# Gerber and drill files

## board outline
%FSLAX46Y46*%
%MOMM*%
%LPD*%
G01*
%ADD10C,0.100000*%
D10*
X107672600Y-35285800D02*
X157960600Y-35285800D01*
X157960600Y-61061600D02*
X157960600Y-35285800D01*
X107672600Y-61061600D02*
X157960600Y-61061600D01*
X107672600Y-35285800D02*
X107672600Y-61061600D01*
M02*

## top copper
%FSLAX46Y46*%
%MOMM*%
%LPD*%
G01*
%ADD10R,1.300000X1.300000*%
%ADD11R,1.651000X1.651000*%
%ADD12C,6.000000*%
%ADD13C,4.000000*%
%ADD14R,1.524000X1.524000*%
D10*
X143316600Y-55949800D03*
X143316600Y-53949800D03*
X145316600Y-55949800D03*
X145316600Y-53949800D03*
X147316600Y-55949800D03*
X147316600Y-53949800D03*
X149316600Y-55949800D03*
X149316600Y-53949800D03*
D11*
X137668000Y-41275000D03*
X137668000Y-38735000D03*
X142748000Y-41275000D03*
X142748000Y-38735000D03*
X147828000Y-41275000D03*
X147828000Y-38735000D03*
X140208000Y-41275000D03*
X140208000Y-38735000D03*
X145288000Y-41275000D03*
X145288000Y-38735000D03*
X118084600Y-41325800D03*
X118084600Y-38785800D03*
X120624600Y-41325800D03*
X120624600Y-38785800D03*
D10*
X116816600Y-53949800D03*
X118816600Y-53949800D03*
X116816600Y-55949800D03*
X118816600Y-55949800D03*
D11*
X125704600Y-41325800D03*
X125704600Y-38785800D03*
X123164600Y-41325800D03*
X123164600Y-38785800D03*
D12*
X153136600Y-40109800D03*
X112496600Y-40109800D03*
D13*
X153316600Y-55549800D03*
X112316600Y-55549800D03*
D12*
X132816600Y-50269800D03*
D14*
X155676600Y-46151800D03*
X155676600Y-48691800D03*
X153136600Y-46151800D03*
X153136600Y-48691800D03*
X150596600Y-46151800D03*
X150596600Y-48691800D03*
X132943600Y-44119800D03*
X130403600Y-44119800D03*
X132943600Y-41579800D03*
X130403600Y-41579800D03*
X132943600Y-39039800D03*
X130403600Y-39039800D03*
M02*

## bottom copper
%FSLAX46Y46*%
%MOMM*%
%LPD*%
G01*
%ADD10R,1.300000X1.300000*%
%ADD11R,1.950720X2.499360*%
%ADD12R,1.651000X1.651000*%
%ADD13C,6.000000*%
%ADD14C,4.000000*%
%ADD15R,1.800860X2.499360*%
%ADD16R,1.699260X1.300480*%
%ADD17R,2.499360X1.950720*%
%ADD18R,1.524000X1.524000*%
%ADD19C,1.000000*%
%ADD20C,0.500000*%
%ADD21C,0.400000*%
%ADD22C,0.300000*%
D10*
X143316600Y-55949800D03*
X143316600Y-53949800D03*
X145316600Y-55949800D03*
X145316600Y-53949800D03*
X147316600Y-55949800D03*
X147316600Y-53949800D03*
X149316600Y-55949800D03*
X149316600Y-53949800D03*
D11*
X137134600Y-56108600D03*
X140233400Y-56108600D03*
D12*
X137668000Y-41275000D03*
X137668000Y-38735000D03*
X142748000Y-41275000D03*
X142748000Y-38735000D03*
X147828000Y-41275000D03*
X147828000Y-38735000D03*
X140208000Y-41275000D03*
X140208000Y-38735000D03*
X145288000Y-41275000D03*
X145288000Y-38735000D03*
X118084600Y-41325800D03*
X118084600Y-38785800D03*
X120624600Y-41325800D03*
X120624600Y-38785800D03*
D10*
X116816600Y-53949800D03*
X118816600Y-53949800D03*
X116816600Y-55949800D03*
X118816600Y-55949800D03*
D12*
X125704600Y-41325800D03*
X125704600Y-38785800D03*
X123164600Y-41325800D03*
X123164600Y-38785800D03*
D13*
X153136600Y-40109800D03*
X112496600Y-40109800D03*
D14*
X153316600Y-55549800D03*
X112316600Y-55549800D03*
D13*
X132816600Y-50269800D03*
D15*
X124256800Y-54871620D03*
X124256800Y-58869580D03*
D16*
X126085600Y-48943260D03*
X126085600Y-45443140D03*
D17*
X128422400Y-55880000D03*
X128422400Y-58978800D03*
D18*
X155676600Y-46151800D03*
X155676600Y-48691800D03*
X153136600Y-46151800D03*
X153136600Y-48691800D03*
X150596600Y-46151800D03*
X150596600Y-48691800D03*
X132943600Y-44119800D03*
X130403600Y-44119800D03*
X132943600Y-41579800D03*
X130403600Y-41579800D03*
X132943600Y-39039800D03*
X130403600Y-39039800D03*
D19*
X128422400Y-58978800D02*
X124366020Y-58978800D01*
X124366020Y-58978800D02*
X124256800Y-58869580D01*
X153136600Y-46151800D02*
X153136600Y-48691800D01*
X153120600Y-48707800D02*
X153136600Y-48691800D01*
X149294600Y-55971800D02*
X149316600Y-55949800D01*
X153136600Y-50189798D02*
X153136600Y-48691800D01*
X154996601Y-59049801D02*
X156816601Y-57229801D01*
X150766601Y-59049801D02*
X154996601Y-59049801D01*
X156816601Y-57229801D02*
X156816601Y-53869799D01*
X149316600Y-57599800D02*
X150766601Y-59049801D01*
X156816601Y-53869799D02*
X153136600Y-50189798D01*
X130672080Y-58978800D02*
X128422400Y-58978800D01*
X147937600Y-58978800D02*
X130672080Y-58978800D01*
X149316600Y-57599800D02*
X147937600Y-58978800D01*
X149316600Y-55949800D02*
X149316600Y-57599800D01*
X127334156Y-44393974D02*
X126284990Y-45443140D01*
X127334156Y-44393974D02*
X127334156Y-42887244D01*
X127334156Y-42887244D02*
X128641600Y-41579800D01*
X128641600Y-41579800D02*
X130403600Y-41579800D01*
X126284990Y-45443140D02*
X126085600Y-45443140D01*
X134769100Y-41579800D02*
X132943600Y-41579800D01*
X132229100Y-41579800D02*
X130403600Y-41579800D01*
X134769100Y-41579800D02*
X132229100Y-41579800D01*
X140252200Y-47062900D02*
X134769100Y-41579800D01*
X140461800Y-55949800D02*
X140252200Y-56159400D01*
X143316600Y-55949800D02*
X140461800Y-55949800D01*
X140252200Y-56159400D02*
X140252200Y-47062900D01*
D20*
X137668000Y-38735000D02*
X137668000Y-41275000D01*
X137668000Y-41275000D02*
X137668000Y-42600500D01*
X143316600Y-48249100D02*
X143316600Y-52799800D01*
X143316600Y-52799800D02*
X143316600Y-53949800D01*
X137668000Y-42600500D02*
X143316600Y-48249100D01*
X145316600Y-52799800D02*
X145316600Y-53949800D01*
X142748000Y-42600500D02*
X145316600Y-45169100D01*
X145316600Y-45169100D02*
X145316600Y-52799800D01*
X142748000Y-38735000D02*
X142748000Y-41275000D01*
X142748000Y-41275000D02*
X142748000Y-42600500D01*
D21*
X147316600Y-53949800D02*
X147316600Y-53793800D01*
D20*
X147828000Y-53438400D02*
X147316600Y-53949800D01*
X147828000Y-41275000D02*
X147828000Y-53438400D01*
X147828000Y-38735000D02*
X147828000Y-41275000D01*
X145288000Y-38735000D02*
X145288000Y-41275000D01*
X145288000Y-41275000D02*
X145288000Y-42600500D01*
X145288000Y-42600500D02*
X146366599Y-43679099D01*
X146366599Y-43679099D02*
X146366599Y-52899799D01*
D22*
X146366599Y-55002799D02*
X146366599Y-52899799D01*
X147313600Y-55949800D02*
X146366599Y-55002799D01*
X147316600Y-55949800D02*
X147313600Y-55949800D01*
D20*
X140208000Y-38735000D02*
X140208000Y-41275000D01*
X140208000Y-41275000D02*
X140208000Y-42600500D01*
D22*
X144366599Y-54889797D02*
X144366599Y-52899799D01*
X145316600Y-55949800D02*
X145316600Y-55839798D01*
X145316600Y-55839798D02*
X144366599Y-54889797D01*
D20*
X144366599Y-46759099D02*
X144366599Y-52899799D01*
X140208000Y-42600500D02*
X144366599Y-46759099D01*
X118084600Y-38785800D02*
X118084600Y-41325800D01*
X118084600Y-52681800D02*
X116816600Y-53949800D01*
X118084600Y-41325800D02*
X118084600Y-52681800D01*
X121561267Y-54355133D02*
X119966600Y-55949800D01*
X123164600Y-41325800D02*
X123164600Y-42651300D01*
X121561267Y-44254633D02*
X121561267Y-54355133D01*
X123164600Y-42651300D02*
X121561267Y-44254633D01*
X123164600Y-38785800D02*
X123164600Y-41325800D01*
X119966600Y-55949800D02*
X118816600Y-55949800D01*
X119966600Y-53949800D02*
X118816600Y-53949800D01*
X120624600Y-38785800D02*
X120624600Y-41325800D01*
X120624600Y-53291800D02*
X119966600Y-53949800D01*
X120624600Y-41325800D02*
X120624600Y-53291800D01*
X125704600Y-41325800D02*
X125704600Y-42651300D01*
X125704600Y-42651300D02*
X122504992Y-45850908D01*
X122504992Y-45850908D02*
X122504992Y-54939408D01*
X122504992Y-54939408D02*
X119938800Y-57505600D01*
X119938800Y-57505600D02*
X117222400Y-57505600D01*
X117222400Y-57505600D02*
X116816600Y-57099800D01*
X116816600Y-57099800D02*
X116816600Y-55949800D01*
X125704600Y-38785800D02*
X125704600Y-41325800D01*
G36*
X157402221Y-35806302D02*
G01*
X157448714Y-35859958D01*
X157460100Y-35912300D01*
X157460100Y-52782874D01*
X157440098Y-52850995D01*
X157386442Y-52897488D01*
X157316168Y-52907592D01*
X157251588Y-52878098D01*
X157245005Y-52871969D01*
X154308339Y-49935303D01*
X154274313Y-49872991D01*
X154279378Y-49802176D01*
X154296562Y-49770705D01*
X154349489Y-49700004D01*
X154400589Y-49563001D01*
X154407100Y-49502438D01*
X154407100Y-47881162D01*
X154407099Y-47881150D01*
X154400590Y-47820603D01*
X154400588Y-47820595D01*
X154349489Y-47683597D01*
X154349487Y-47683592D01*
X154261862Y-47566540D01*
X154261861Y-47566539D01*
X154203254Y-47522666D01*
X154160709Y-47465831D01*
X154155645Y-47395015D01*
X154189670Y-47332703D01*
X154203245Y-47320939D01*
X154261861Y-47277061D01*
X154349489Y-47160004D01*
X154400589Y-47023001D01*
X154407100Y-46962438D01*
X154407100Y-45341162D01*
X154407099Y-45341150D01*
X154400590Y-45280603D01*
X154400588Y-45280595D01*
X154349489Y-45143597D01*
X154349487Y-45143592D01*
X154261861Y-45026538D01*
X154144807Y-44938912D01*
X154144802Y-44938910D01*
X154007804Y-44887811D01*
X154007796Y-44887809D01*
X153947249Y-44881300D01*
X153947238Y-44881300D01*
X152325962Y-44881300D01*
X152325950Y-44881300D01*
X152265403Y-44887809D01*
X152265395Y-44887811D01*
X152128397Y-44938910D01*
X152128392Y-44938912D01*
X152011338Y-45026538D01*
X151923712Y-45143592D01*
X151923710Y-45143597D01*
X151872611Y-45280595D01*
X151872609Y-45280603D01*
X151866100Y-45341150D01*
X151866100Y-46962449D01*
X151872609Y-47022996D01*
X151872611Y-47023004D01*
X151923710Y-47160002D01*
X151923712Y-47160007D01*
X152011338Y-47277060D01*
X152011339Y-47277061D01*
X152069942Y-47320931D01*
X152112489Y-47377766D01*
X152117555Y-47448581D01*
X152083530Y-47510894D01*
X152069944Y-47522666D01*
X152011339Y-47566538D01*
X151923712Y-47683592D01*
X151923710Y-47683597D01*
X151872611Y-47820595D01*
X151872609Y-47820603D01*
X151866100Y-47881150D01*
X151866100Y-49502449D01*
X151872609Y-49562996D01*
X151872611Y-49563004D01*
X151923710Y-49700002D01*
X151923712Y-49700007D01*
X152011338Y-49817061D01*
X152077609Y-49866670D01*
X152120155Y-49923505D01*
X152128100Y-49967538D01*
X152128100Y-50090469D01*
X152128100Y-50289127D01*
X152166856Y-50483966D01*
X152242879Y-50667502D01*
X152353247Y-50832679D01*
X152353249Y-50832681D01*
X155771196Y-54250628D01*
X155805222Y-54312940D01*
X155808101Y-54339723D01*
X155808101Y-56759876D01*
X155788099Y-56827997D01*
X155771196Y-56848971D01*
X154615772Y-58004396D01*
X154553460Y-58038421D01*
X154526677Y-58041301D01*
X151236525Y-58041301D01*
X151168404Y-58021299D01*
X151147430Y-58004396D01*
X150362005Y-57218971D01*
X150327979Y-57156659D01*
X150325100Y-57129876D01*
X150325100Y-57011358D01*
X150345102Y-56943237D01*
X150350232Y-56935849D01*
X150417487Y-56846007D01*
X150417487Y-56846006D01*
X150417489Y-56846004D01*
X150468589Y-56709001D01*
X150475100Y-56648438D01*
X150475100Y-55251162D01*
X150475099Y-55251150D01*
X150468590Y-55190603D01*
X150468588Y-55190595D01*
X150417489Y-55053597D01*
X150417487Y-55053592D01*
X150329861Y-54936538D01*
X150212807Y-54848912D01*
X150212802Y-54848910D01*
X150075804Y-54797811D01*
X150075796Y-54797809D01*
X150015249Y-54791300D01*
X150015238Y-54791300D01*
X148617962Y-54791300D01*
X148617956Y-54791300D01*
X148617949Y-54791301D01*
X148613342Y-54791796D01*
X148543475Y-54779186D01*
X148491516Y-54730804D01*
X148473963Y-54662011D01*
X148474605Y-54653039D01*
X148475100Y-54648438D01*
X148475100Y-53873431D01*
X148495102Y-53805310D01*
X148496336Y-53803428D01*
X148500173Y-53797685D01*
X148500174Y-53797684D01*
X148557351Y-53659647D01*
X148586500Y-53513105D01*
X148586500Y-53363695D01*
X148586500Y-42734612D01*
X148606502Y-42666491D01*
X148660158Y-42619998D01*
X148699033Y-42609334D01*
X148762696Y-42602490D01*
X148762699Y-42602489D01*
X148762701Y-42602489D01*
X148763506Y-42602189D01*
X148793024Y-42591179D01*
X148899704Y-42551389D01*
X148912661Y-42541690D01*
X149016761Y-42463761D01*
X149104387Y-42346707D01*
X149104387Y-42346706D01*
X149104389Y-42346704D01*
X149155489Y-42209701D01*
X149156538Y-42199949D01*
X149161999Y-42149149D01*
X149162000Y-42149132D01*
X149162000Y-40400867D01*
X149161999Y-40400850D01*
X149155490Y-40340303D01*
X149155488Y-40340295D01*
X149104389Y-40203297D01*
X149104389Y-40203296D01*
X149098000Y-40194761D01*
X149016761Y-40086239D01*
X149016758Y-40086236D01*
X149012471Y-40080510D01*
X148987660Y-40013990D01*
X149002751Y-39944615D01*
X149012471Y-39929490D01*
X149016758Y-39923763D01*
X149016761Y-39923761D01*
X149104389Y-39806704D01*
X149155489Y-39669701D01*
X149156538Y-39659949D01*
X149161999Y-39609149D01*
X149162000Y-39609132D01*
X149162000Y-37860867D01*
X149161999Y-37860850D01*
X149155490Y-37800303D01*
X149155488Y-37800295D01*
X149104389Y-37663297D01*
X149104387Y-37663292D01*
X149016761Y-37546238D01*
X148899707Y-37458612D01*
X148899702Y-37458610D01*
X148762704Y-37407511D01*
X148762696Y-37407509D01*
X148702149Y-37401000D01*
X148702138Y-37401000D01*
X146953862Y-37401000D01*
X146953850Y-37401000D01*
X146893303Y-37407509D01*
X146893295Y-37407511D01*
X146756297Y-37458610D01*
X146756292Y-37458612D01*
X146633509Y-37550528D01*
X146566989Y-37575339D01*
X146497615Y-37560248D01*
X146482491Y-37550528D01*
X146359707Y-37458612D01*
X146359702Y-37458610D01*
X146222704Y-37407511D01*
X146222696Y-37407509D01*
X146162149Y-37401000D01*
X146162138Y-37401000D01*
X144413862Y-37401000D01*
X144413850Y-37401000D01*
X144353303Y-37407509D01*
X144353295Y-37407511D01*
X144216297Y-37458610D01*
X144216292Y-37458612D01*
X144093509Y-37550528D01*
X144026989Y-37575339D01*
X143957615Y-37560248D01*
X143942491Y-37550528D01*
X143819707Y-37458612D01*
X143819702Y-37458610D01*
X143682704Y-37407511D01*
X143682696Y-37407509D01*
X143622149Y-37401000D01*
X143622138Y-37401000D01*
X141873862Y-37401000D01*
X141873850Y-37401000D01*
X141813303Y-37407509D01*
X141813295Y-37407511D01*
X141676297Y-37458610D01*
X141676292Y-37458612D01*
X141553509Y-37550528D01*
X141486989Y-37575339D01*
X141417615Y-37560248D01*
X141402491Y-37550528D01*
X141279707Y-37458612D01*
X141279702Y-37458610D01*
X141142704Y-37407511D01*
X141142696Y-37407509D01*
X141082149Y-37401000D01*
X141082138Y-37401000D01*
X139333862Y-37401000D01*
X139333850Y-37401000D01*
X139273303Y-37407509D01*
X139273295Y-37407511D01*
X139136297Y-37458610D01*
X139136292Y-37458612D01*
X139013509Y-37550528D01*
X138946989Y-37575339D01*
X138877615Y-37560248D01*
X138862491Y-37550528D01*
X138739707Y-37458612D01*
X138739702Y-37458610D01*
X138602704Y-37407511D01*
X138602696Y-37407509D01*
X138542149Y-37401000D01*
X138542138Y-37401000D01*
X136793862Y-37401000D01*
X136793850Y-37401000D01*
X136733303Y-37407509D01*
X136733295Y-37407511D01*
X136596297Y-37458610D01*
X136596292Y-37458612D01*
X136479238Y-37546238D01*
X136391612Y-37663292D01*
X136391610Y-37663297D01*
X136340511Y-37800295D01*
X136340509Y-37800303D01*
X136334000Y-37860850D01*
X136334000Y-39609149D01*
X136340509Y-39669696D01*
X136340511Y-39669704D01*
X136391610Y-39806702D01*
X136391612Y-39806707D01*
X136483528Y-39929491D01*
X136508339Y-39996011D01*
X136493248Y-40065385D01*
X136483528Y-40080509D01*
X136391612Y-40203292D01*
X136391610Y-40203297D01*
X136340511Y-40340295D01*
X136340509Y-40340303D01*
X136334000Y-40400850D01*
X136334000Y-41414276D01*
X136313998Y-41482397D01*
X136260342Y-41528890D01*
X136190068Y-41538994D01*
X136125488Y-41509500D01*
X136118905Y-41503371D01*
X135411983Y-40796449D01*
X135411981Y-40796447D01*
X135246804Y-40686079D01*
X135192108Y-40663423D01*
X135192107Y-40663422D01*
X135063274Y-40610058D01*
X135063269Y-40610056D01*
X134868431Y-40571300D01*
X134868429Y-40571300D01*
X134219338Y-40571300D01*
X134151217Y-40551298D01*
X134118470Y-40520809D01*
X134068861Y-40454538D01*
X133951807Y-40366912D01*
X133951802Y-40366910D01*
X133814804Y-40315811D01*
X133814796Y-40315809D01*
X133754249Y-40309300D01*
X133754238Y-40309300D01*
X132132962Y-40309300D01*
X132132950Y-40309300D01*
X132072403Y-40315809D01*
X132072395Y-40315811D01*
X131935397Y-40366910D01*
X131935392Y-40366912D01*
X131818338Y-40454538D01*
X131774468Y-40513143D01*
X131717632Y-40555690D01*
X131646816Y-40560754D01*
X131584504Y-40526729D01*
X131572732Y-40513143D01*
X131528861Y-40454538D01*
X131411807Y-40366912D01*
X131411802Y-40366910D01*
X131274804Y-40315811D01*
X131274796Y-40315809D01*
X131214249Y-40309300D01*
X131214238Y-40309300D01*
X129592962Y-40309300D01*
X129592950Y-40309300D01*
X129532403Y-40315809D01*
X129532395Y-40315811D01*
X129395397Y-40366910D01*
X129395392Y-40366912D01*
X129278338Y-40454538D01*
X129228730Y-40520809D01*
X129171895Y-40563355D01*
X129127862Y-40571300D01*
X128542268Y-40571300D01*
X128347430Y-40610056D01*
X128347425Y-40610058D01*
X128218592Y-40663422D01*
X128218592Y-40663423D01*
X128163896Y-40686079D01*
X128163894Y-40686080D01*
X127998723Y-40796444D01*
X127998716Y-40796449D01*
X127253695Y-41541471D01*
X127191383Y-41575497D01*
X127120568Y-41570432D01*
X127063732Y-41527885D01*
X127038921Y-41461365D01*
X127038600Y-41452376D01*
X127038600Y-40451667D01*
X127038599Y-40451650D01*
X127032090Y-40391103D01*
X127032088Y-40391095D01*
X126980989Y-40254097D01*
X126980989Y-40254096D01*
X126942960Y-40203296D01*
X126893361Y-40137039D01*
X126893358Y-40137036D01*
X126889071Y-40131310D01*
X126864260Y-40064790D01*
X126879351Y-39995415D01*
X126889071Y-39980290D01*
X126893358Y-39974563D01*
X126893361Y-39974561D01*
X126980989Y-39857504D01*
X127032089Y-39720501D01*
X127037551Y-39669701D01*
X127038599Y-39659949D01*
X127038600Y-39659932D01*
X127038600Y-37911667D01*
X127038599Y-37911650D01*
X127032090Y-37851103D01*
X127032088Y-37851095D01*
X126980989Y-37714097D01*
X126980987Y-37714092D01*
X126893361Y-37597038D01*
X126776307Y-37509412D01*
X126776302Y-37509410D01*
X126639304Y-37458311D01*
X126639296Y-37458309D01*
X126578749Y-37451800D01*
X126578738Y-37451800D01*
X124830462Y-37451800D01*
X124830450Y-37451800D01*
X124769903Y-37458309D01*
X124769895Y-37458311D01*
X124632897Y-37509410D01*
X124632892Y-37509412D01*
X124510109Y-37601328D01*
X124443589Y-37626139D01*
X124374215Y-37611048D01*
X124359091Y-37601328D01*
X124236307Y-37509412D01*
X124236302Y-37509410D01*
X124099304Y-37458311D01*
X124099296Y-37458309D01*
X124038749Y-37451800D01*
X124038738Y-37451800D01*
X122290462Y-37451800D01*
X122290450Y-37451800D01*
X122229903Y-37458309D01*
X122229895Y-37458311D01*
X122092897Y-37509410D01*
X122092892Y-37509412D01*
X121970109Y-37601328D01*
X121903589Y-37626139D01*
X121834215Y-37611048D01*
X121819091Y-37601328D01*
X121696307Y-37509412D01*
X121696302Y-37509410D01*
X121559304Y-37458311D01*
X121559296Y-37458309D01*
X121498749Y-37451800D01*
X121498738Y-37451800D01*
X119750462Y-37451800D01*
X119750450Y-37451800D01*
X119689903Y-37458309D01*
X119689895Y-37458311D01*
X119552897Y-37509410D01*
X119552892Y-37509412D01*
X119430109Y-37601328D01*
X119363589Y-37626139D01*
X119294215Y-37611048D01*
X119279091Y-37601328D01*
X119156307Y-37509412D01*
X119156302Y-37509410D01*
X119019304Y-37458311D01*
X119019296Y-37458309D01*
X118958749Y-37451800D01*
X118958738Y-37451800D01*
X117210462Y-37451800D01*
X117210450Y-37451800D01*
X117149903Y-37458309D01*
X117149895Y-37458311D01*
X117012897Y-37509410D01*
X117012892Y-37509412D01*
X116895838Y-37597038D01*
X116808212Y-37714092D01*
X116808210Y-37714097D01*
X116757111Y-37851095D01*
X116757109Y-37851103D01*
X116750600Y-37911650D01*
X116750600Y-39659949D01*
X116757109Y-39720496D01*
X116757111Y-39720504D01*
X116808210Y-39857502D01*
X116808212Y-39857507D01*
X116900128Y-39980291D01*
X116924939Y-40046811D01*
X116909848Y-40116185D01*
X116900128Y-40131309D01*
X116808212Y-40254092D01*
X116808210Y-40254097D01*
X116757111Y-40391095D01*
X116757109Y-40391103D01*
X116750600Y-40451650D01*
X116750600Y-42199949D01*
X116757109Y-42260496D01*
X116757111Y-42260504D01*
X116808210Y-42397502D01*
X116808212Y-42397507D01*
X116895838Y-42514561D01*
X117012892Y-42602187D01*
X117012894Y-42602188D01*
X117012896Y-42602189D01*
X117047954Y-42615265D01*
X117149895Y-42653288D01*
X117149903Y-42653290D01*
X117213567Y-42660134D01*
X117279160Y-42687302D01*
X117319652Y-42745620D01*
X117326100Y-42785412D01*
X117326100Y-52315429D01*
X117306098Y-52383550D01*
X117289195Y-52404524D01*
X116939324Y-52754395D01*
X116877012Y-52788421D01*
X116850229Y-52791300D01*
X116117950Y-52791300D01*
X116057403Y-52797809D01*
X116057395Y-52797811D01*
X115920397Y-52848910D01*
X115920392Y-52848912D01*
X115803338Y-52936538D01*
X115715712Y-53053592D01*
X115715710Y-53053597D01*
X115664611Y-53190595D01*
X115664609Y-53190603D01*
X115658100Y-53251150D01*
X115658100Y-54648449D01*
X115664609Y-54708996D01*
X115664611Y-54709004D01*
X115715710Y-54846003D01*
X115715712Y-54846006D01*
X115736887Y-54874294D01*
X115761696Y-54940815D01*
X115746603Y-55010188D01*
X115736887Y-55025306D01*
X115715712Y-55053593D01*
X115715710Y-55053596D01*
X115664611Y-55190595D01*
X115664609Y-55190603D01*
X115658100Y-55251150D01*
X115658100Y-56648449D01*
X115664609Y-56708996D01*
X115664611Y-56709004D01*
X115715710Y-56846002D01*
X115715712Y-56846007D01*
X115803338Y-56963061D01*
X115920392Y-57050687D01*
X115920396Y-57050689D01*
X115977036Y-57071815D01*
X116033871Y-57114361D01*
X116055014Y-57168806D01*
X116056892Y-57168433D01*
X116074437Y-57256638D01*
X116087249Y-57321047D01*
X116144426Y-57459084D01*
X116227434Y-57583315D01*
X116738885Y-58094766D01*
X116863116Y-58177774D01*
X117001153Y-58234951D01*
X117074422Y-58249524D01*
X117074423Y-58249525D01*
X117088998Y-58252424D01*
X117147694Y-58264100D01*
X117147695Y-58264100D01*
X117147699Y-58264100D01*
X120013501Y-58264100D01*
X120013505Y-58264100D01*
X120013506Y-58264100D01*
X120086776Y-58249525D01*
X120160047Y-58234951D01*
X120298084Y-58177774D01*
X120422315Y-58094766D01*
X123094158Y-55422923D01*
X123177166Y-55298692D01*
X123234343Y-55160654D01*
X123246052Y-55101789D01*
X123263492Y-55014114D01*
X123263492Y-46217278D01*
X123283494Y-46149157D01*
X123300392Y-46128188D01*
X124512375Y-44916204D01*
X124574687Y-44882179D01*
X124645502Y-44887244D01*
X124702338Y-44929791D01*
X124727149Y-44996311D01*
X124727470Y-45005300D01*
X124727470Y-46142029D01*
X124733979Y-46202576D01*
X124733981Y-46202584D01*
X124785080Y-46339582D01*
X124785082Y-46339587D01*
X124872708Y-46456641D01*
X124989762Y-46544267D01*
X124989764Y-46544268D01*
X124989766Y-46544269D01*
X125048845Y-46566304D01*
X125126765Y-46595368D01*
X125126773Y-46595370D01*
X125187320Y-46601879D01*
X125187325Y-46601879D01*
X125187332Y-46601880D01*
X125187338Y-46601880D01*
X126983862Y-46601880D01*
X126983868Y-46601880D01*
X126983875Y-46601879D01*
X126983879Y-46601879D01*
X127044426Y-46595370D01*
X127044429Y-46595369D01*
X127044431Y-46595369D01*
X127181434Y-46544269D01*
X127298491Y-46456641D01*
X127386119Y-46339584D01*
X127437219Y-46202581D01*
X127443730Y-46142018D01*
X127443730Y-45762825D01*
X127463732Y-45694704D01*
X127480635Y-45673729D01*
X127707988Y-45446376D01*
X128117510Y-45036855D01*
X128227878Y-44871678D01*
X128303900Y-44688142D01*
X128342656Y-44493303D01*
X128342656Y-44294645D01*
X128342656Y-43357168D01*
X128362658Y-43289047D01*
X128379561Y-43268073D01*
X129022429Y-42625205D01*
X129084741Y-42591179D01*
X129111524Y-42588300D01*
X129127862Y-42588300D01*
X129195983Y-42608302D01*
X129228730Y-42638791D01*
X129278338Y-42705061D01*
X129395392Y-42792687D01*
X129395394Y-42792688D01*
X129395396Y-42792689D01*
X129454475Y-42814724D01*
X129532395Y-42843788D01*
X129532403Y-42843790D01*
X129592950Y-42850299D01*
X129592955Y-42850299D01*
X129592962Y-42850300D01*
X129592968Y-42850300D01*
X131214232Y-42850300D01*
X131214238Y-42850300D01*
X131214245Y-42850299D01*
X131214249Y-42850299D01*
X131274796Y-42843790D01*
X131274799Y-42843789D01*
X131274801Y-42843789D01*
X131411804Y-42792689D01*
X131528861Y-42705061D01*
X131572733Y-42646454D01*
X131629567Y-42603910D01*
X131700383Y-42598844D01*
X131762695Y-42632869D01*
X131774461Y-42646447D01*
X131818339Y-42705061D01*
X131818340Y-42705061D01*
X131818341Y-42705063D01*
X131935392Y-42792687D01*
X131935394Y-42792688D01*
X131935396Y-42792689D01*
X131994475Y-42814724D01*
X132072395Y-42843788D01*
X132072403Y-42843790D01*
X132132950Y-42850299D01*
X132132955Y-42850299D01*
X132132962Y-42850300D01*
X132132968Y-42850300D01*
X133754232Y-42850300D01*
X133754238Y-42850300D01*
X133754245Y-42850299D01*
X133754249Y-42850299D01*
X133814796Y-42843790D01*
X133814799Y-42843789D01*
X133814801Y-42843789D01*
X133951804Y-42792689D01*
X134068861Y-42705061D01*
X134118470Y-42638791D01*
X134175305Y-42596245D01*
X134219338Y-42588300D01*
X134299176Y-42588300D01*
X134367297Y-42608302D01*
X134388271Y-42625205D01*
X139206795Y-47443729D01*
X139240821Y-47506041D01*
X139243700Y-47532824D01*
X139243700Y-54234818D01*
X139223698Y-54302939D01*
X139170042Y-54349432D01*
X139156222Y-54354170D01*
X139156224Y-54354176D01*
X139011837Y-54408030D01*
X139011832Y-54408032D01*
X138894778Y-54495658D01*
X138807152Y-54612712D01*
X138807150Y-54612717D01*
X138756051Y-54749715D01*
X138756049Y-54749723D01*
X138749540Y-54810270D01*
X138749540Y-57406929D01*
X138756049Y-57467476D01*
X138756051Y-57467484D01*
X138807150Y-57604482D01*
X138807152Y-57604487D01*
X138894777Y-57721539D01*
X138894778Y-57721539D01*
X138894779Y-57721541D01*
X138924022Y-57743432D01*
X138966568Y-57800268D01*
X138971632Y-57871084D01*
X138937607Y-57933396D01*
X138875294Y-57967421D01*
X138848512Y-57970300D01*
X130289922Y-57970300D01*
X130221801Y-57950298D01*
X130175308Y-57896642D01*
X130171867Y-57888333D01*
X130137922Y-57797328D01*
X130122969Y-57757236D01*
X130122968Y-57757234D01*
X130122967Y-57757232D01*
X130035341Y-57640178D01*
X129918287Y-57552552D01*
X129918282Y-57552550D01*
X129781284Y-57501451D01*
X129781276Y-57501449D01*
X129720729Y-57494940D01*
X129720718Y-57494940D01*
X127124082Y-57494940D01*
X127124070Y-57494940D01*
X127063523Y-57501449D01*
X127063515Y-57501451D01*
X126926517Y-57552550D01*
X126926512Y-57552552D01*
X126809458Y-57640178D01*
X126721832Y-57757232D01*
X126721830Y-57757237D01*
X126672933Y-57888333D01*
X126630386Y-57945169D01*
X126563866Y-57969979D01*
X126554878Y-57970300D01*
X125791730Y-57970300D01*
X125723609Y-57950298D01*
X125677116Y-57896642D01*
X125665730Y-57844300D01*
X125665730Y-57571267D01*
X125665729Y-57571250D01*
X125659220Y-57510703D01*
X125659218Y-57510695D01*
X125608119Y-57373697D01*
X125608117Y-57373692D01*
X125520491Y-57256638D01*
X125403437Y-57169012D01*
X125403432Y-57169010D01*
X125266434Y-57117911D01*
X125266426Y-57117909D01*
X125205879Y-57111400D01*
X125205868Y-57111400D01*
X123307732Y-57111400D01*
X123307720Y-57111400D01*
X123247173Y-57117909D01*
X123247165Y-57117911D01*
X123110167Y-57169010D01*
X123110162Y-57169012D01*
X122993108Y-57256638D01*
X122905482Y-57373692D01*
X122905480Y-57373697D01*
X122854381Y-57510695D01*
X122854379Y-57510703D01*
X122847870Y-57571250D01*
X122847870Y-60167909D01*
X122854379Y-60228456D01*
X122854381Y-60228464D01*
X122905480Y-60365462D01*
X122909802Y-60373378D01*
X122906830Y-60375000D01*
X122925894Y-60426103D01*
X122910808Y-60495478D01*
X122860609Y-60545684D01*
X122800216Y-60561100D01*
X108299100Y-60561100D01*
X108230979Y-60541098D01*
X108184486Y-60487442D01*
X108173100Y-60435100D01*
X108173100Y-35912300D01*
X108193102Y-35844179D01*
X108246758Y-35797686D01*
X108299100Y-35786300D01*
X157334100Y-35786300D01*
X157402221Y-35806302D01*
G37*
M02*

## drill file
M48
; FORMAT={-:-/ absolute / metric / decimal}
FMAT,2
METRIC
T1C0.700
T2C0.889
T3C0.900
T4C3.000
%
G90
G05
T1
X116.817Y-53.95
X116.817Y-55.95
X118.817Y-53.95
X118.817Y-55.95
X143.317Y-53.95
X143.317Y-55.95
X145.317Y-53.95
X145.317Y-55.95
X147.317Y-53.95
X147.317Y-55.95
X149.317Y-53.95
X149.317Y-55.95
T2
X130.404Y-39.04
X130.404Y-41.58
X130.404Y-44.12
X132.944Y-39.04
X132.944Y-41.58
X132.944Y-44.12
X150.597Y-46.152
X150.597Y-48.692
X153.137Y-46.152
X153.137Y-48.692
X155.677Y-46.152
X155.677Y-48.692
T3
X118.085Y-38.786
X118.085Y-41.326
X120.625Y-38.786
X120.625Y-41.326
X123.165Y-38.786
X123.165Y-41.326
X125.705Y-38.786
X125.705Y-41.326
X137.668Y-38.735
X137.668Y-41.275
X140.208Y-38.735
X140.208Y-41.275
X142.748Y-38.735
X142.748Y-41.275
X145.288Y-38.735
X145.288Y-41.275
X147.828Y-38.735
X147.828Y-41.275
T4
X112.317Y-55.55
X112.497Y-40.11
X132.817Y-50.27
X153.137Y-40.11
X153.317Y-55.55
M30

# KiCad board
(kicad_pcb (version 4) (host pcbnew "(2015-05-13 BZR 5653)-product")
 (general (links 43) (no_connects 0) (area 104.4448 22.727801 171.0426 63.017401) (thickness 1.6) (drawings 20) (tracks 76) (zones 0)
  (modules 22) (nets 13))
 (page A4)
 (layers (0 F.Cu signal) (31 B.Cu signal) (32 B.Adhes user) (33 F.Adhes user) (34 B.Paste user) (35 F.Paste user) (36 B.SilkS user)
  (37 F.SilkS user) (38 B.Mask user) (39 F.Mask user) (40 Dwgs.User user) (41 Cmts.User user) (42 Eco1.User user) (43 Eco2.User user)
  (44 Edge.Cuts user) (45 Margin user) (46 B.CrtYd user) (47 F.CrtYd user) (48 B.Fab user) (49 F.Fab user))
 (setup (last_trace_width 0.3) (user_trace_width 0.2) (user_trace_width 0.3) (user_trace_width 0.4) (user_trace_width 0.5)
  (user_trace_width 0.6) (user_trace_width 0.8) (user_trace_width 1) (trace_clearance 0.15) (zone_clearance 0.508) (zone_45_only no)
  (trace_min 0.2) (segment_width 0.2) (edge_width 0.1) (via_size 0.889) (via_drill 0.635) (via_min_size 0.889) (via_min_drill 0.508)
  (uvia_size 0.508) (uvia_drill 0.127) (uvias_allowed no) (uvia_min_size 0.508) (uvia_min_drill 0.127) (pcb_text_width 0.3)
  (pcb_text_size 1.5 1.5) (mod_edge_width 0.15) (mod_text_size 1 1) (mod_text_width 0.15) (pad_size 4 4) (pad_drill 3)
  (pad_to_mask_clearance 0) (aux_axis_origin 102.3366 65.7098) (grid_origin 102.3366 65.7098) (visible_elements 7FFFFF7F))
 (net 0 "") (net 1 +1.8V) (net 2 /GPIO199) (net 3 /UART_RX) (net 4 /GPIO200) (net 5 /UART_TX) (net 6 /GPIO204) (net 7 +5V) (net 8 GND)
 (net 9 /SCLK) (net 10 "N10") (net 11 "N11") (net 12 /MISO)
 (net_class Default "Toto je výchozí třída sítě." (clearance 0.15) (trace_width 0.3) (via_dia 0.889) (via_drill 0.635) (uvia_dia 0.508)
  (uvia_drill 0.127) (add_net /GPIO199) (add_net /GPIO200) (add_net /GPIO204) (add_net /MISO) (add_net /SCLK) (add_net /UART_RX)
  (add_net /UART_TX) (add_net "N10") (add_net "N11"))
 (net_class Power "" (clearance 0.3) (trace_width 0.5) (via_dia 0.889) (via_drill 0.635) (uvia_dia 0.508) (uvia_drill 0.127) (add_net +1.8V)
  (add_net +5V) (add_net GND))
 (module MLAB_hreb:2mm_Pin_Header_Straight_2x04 (layer F.Cu) (at 146.3166 54.9498 90)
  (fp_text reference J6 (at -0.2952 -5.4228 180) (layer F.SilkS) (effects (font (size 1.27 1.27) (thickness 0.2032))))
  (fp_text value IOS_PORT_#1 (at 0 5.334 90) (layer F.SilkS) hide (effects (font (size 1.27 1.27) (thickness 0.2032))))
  (pad 1 thru_hole rect (at -1 -3 90) (size 1.3 1.3) (drill 0.7) (layers *.Cu *.Mask F.SilkS) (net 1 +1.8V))
  (pad 2 thru_hole rect (at 1 -3 90) (size 1.3 1.3) (drill 0.7) (layers *.Cu *.Mask F.SilkS) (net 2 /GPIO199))
  (pad 3 thru_hole rect (at -1 -1 90) (size 1.3 1.3) (drill 0.7) (layers *.Cu *.Mask F.SilkS) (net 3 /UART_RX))
  (pad 4 thru_hole rect (at 1 -1 90) (size 1.3 1.3) (drill 0.7) (layers *.Cu *.Mask F.SilkS) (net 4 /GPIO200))
  (pad 5 thru_hole rect (at -1 1 90) (size 1.3 1.3) (drill 0.7) (layers *.Cu *.Mask F.SilkS) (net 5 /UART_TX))
  (pad 6 thru_hole rect (at 1 1 90) (size 1.3 1.3) (drill 0.7) (layers *.Cu *.Mask F.SilkS) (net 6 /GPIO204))
  (pad 7 thru_hole rect (at -1 3 90) (size 1.3 1.3) (drill 0.7) (layers *.Cu *.Mask F.SilkS) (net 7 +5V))
  (pad 8 thru_hole rect (at 1 3 90) (size 1.3 1.3) (drill 0.7) (layers *.Cu *.Mask F.SilkS) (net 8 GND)))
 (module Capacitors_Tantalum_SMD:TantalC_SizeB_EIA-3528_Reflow (layer B.Cu) (at 138.684 56.1086 180)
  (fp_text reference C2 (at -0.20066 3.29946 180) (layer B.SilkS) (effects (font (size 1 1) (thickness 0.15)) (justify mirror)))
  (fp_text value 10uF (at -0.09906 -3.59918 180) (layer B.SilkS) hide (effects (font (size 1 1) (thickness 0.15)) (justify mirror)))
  (pad 2 smd rect (at 1.5494 0 180) (size 1.95072 2.49936) (layers B.Cu B.Paste B.Mask) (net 8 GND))
  (pad 1 smd rect (at -1.5494 0 180) (size 1.95072 2.49936) (layers B.Cu B.Paste B.Mask) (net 1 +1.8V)))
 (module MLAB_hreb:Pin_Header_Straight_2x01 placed (layer F.Cu) (at 137.668 40.005)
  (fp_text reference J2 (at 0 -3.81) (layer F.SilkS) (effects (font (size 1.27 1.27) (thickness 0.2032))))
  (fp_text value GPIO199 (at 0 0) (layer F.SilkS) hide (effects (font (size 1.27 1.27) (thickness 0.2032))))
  (pad 2 thru_hole rect (at 0 1.27) (size 1.651 1.651) (drill 0.9) (layers *.Cu *.Mask F.SilkS) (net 2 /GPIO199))
  (pad 1 thru_hole rect (at 0 -1.27) (size 1.651 1.651) (drill 0.9) (layers *.Cu *.Mask F.SilkS) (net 2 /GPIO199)))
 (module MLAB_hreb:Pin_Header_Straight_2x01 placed (layer F.Cu) (at 142.748 40.005)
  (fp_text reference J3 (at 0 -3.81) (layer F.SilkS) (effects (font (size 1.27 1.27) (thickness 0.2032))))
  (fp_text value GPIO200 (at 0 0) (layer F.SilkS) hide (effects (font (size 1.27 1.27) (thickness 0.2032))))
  (pad 2 thru_hole rect (at 0 1.27) (size 1.651 1.651) (drill 0.9) (layers *.Cu *.Mask F.SilkS) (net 4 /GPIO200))
  (pad 1 thru_hole rect (at 0 -1.27) (size 1.651 1.651) (drill 0.9) (layers *.Cu *.Mask F.SilkS) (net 4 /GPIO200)))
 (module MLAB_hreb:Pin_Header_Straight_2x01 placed (layer F.Cu) (at 147.828 40.005)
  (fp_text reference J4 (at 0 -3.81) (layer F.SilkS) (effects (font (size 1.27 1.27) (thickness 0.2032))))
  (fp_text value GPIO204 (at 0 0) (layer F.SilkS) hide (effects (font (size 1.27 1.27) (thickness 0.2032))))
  (pad 2 thru_hole rect (at 0 1.27) (size 1.651 1.651) (drill 0.9) (layers *.Cu *.Mask F.SilkS) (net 6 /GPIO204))
  (pad 1 thru_hole rect (at 0 -1.27) (size 1.651 1.651) (drill 0.9) (layers *.Cu *.Mask F.SilkS) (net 6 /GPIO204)))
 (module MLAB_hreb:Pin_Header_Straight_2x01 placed (layer F.Cu) (at 140.208 40.005)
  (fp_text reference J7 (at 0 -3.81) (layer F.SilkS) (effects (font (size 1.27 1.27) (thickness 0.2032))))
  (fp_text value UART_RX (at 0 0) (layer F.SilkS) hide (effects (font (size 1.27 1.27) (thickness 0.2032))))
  (pad 2 thru_hole rect (at 0 1.27) (size 1.651 1.651) (drill 0.9) (layers *.Cu *.Mask F.SilkS) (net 3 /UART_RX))
  (pad 1 thru_hole rect (at 0 -1.27) (size 1.651 1.651) (drill 0.9) (layers *.Cu *.Mask F.SilkS) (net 3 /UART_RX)))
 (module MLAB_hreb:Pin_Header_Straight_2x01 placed (layer F.Cu) (at 145.288 40.005)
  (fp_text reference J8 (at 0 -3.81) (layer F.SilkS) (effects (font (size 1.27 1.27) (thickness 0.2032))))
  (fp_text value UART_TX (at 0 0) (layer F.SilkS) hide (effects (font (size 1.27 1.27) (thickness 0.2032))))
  (pad 2 thru_hole rect (at 0 1.27) (size 1.651 1.651) (drill 0.9) (layers *.Cu *.Mask F.SilkS) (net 5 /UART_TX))
  (pad 1 thru_hole rect (at 0 -1.27) (size 1.651 1.651) (drill 0.9) (layers *.Cu *.Mask F.SilkS) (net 5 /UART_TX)))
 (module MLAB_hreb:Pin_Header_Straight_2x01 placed (layer F.Cu) (at 118.0846 40.0558)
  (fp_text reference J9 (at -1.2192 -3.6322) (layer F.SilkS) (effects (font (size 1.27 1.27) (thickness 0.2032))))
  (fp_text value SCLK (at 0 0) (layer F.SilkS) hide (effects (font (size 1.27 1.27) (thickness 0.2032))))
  (pad 2 thru_hole rect (at 0 1.27) (size 1.651 1.651) (drill 0.9) (layers *.Cu *.Mask F.SilkS) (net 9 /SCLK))
  (pad 1 thru_hole rect (at 0 -1.27) (size 1.651 1.651) (drill 0.9) (layers *.Cu *.Mask F.SilkS) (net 9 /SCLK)))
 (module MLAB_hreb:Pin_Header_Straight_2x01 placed (layer F.Cu) (at 120.6246 40.0558)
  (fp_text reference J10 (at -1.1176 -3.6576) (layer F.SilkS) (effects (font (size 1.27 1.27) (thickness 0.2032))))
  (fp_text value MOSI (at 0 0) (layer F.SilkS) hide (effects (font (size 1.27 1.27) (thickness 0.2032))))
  (pad 2 thru_hole rect (at 0 1.27) (size 1.651 1.651) (drill 0.9) (layers *.Cu *.Mask F.SilkS) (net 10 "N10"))
  (pad 1 thru_hole rect (at 0 -1.27) (size 1.651 1.651) (drill 0.9) (layers *.Cu *.Mask F.SilkS) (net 10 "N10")))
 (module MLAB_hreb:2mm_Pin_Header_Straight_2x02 (layer F.Cu) (at 117.8166 54.9498)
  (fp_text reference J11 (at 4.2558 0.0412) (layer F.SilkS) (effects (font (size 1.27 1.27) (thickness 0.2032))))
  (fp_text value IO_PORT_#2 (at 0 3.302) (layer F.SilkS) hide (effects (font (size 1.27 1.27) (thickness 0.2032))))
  (pad 1 thru_hole rect (at -1 -1) (size 1.3 1.3) (drill 0.7) (layers *.Cu *.Mask F.SilkS) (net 9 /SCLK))
  (pad 2 thru_hole rect (at 1 -1) (size 1.3 1.3) (drill 0.7) (layers *.Cu *.Mask F.SilkS) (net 10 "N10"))
  (pad 3 thru_hole rect (at -1 1) (size 1.3 1.3) (drill 0.7) (layers *.Cu *.Mask F.SilkS) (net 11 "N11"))
  (pad 4 thru_hole rect (at 1 1) (size 1.3 1.3) (drill 0.7) (layers *.Cu *.Mask F.SilkS) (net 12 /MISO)))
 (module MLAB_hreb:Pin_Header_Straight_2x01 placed (layer F.Cu) (at 125.7046 40.0558)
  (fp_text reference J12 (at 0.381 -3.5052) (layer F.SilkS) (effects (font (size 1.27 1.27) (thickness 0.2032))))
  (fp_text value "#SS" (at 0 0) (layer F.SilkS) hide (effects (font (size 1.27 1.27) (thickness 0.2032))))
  (pad 2 thru_hole rect (at 0 1.27) (size 1.651 1.651) (drill 0.9) (layers *.Cu *.Mask F.SilkS) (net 11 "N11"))
  (pad 1 thru_hole rect (at 0 -1.27) (size 1.651 1.651) (drill 0.9) (layers *.Cu *.Mask F.SilkS) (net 11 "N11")))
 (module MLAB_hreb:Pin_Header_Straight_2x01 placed (layer F.Cu) (at 123.1646 40.0558)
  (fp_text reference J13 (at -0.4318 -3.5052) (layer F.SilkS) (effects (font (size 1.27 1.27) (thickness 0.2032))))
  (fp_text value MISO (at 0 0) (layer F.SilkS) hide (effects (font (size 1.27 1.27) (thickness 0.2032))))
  (pad 2 thru_hole rect (at 0 1.27) (size 1.651 1.651) (drill 0.9) (layers *.Cu *.Mask F.SilkS) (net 12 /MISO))
  (pad 1 thru_hole rect (at 0 -1.27) (size 1.651 1.651) (drill 0.9) (layers *.Cu *.Mask F.SilkS) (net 12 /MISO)))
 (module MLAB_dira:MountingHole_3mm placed (layer F.Cu) (at 153.1366 40.1098)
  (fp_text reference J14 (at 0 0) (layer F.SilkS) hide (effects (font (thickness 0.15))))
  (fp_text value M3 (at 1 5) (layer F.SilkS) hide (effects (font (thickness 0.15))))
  (pad 1 thru_hole circle (at 0 0) (size 6 6) (drill 3) (layers *.Cu *.Adhes *.Mask) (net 8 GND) (clearance 1) (zone_connect 2)))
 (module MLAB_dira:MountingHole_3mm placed (layer F.Cu) (at 112.4966 40.1098)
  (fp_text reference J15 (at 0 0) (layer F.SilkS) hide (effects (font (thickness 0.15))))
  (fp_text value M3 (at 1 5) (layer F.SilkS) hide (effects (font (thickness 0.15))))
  (pad 1 thru_hole circle (at 0 0) (size 6 6) (drill 3) (layers *.Cu *.Adhes *.Mask) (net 8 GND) (clearance 1) (zone_connect 2)))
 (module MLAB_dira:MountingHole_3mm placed (layer F.Cu) (at 153.3166 55.5498)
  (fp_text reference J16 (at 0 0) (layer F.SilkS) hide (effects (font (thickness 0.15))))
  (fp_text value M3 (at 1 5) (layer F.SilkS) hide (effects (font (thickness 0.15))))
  (pad 1 thru_hole circle (at 0 0) (size 4 4) (drill 3) (layers *.Cu *.Adhes *.Mask) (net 8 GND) (clearance 1) (zone_connect 2)))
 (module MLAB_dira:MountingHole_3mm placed (layer F.Cu) (at 112.3166 55.5498)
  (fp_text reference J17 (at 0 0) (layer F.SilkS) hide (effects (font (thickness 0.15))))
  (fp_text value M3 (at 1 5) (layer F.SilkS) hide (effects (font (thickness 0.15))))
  (pad 1 thru_hole circle (at 0 0) (size 4 4) (drill 3) (layers *.Cu *.Adhes *.Mask) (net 8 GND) (clearance 1) (zone_connect 2)))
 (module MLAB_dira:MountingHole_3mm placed (layer F.Cu) (at 132.8166 50.2698)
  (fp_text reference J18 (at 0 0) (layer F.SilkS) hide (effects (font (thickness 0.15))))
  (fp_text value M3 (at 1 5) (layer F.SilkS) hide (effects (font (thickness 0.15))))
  (pad 1 thru_hole circle (at 0 0) (size 6 6) (drill 3) (layers *.Cu *.Adhes *.Mask) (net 8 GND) (clearance 1) (zone_connect 2)))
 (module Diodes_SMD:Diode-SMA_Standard (layer B.Cu) (at 124.2568 56.8706 270)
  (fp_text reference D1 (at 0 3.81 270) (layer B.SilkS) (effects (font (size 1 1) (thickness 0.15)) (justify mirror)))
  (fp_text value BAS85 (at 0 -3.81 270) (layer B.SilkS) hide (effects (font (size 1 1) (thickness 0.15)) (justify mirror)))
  (pad 1 smd rect (at -1.99898 0 270) (size 2.49936 1.80086) (layers B.Cu B.Paste B.Mask) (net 8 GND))
  (pad 2 smd rect (at 1.99898 0 270) (size 2.49936 1.80086) (layers B.Cu B.Paste B.Mask) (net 7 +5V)))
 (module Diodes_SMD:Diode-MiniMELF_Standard (layer B.Cu) (at 126.0856 47.1932 90)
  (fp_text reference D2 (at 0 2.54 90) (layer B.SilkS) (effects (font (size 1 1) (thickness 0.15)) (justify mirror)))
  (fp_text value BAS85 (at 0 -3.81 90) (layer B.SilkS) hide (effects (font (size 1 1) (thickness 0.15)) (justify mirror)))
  (pad 1 smd rect (at -1.75006 0 90) (size 1.30048 1.69926) (layers B.Cu B.Paste B.Mask) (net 8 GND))
  (pad 2 smd rect (at 1.75006 0 90) (size 1.30048 1.69926) (layers B.Cu B.Paste B.Mask) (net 1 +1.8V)))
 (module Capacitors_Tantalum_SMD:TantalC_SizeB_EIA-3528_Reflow (layer B.Cu) (at 128.4224 57.4294 90)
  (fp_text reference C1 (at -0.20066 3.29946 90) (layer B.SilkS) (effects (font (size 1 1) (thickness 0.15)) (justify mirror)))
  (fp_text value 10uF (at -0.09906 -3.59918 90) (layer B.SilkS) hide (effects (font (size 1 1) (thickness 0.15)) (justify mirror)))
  (pad 2 smd rect (at 1.5494 0 90) (size 1.95072 2.49936) (layers B.Cu B.Paste B.Mask) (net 8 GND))
  (pad 1 smd rect (at -1.5494 0 90) (size 1.95072 2.49936) (layers B.Cu B.Paste B.Mask) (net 7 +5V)))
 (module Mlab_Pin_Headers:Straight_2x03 (layer F.Cu) (at 153.1366 47.4218 270)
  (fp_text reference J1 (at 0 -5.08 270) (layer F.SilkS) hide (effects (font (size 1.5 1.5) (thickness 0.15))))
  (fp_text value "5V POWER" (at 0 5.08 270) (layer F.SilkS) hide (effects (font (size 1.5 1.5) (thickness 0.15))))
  (pad 1 thru_hole rect (at -1.27 -2.54 270) (size 1.524 1.524) (drill 0.889) (layers *.Cu *.Mask F.SilkS) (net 8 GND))
  (pad 2 thru_hole rect (at 1.27 -2.54 270) (size 1.524 1.524) (drill 0.889) (layers *.Cu *.Mask F.SilkS) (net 8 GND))
  (pad 3 thru_hole rect (at -1.27 0 270) (size 1.524 1.524) (drill 0.889) (layers *.Cu *.Mask F.SilkS) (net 7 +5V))
  (pad 4 thru_hole rect (at 1.27 0 270) (size 1.524 1.524) (drill 0.889) (layers *.Cu *.Mask F.SilkS) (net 7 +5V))
  (pad 5 thru_hole rect (at -1.27 2.54 270) (size 1.524 1.524) (drill 0.889) (layers *.Cu *.Mask F.SilkS) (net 8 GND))
  (pad 6 thru_hole rect (at 1.27 2.54 270) (size 1.524 1.524) (drill 0.889) (layers *.Cu *.Mask F.SilkS) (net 8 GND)))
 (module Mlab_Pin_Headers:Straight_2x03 (layer F.Cu) (at 131.6736 41.5798 180)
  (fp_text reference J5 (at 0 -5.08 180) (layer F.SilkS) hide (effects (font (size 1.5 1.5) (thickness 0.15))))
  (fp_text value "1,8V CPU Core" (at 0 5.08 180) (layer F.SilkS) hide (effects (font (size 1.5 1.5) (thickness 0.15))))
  (pad 1 thru_hole rect (at -1.27 -2.54 180) (size 1.524 1.524) (drill 0.889) (layers *.Cu *.Mask F.SilkS) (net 8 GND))
  (pad 2 thru_hole rect (at 1.27 -2.54 180) (size 1.524 1.524) (drill 0.889) (layers *.Cu *.Mask F.SilkS) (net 8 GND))
  (pad 3 thru_hole rect (at -1.27 0 180) (size 1.524 1.524) (drill 0.889) (layers *.Cu *.Mask F.SilkS) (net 1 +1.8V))
  (pad 4 thru_hole rect (at 1.27 0 180) (size 1.524 1.524) (drill 0.889) (layers *.Cu *.Mask F.SilkS) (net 1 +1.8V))
  (pad 5 thru_hole rect (at -1.27 2.54 180) (size 1.524 1.524) (drill 0.889) (layers *.Cu *.Mask F.SilkS) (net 8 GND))
  (pad 6 thru_hole rect (at 1.27 2.54 180) (size 1.524 1.524) (drill 0.889) (layers *.Cu *.Mask F.SilkS) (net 8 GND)))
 (gr_line (start 107.6726 35.2858) (end 157.9606 35.2858) (angle 90) (layer Edge.Cuts) (width 0.1))
 (gr_line (start 157.9606 61.0616) (end 157.9606 35.2858) (angle 90) (layer Edge.Cuts) (width 0.1))
 (gr_line (start 107.6726 61.0616) (end 157.9606 61.0616) (angle 90) (layer Edge.Cuts) (width 0.1))
 (gr_line (start 107.6726 35.2858) (end 107.6726 61.0616) (angle 90) (layer Edge.Cuts) (width 0.1))
 (segment (start 128.4224 58.9788) (end 124.36602 58.9788) (width 1) (layer B.Cu) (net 7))
 (segment (start 124.36602 58.9788) (end 124.2568 58.86958) (width 1) (layer B.Cu) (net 7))
 (segment (start 153.1366 46.1518) (end 153.1366 48.6918) (width 1) (layer B.Cu) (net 7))
 (segment (start 153.1206 48.7078) (end 153.1366 48.6918) (width 1) (layer B.Cu) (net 7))
 (segment (start 149.2946 55.9718) (end 149.3166 55.9498) (width 1) (layer B.Cu) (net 7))
 (segment (start 153.1366 50.189798) (end 153.1366 48.6918) (width 1) (layer B.Cu) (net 7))
 (segment (start 154.996601 59.049801) (end 156.816601 57.229801) (width 1) (layer B.Cu) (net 7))
 (segment (start 150.766601 59.049801) (end 154.996601 59.049801) (width 1) (layer B.Cu) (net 7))
 (segment (start 156.816601 57.229801) (end 156.816601 53.869799) (width 1) (layer B.Cu) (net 7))
 (segment (start 149.3166 57.5998) (end 150.766601 59.049801) (width 1) (layer B.Cu) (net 7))
 (segment (start 156.816601 53.869799) (end 153.1366 50.189798) (width 1) (layer B.Cu) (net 7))
 (segment (start 130.67208 58.9788) (end 128.4224 58.9788) (width 1) (layer B.Cu) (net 7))
 (segment (start 147.9376 58.9788) (end 130.67208 58.9788) (width 1) (layer B.Cu) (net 7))
 (segment (start 149.3166 57.5998) (end 147.9376 58.9788) (width 1) (layer B.Cu) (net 7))
 (segment (start 149.3166 55.9498) (end 149.3166 57.5998) (width 1) (layer B.Cu) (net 7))
 (segment (start 127.334156 44.393974) (end 126.28499 45.44314) (width 1) (layer B.Cu) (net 1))
 (segment (start 127.334156 44.393974) (end 127.334156 42.887244) (width 1) (layer B.Cu) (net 1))
 (segment (start 127.334156 42.887244) (end 128.6416 41.5798) (width 1) (layer B.Cu) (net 1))
 (segment (start 128.6416 41.5798) (end 130.4036 41.5798) (width 1) (layer B.Cu) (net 1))
 (segment (start 126.28499 45.44314) (end 126.0856 45.44314) (width 1) (layer B.Cu) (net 1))
 (segment (start 134.7691 41.5798) (end 132.9436 41.5798) (width 1) (layer B.Cu) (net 1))
 (segment (start 132.2291 41.5798) (end 130.4036 41.5798) (width 1) (layer B.Cu) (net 1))
 (segment (start 134.7691 41.5798) (end 132.2291 41.5798) (width 1) (layer B.Cu) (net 1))
 (segment (start 140.2522 47.0629) (end 134.7691 41.5798) (width 1) (layer B.Cu) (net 1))
 (segment (start 140.4618 55.9498) (end 140.2522 56.1594) (width 1) (layer B.Cu) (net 1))
 (segment (start 143.3166 55.9498) (end 140.4618 55.9498) (width 1) (layer B.Cu) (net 1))
 (segment (start 140.2522 56.1594) (end 140.2522 47.0629) (width 1) (layer B.Cu) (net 1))
 (segment (start 137.668 38.735) (end 137.668 41.275) (width 0.5) (layer B.Cu) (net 2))
 (segment (start 137.668 41.275) (end 137.668 42.6005) (width 0.5) (layer B.Cu) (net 2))
 (segment (start 143.3166 48.2491) (end 143.3166 52.7998) (width 0.5) (layer B.Cu) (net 2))
 (segment (start 143.3166 52.7998) (end 143.3166 53.9498) (width 0.5) (layer B.Cu) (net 2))
 (segment (start 137.668 42.6005) (end 143.3166 48.2491) (width 0.5) (layer B.Cu) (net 2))
 (segment (start 145.3166 52.7998) (end 145.3166 53.9498) (width 0.5) (layer B.Cu) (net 4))
 (segment (start 142.748 42.6005) (end 145.3166 45.1691) (width 0.5) (layer B.Cu) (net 4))
 (segment (start 145.3166 45.1691) (end 145.3166 52.7998) (width 0.5) (layer B.Cu) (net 4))
 (segment (start 142.748 38.735) (end 142.748 41.275) (width 0.5) (layer B.Cu) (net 4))
 (segment (start 142.748 41.275) (end 142.748 42.6005) (width 0.5) (layer B.Cu) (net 4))
 (segment (start 147.3166 53.9498) (end 147.3166 53.7938) (width 0.4) (layer B.Cu) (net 6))
 (segment (start 147.828 53.4384) (end 147.3166 53.9498) (width 0.5) (layer B.Cu) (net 6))
 (segment (start 147.828 41.275) (end 147.828 53.4384) (width 0.5) (layer B.Cu) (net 6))
 (segment (start 147.828 38.735) (end 147.828 41.275) (width 0.5) (layer B.Cu) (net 6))
 (segment (start 145.288 38.735) (end 145.288 41.275) (width 0.5) (layer B.Cu) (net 5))
 (segment (start 145.288 41.275) (end 145.288 42.6005) (width 0.5) (layer B.Cu) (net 5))
 (segment (start 145.288 42.6005) (end 146.366599 43.679099) (width 0.5) (layer B.Cu) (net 5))
 (segment (start 146.366599 43.679099) (end 146.366599 52.899799) (width 0.5) (layer B.Cu) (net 5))
 (segment (start 146.366599 55.002799) (end 146.366599 52.899799) (width 0.3) (layer B.Cu) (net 5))
 (segment (start 147.3136 55.9498) (end 146.366599 55.002799) (width 0.3) (layer B.Cu) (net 5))
 (segment (start 147.3166 55.9498) (end 147.3136 55.9498) (width 0.3) (layer B.Cu) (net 5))
 (segment (start 140.208 38.735) (end 140.208 41.275) (width 0.5) (layer B.Cu) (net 3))
 (segment (start 140.208 41.275) (end 140.208 42.6005) (width 0.5) (layer B.Cu) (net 3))
 (segment (start 144.366599 54.889797) (end 144.366599 52.899799) (width 0.3) (layer B.Cu) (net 3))
 (segment (start 145.3166 55.9498) (end 145.3166 55.839798) (width 0.3) (layer B.Cu) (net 3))
 (segment (start 145.3166 55.839798) (end 144.366599 54.889797) (width 0.3) (layer B.Cu) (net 3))
 (segment (start 144.366599 46.759099) (end 144.366599 52.899799) (width 0.5) (layer B.Cu) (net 3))
 (segment (start 140.208 42.6005) (end 144.366599 46.759099) (width 0.5) (layer B.Cu) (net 3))
 (segment (start 118.0846 38.7858) (end 118.0846 41.3258) (width 0.5) (layer B.Cu) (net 9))
 (segment (start 118.0846 52.6818) (end 116.8166 53.9498) (width 0.5) (layer B.Cu) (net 9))
 (segment (start 118.0846 41.3258) (end 118.0846 52.6818) (width 0.5) (layer B.Cu) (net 9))
 (segment (start 121.561267 54.355133) (end 119.9666 55.9498) (width 0.5) (layer B.Cu) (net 12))
 (segment (start 123.1646 41.3258) (end 123.1646 42.6513) (width 0.5) (layer B.Cu) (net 12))
 (segment (start 121.561267 44.254633) (end 121.561267 54.355133) (width 0.5) (layer B.Cu) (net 12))
 (segment (start 123.1646 42.6513) (end 121.561267 44.254633) (width 0.5) (layer B.Cu) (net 12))
 (segment (start 123.1646 38.7858) (end 123.1646 41.3258) (width 0.5) (layer B.Cu) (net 12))
 (segment (start 119.9666 55.9498) (end 118.8166 55.9498) (width 0.5) (layer B.Cu) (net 12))
 (segment (start 119.9666 53.9498) (end 118.8166 53.9498) (width 0.5) (layer B.Cu) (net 10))
 (segment (start 120.6246 38.7858) (end 120.6246 41.3258) (width 0.5) (layer B.Cu) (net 10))
 (segment (start 120.6246 53.2918) (end 119.9666 53.9498) (width 0.5) (layer B.Cu) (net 10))
 (segment (start 120.6246 41.3258) (end 120.6246 53.2918) (width 0.5) (layer B.Cu) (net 10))
 (segment (start 125.7046 41.3258) (end 125.7046 42.6513) (width 0.5) (layer B.Cu) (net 11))
 (segment (start 125.7046 42.6513) (end 122.504992 45.850908) (width 0.5) (layer B.Cu) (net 11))
 (segment (start 122.504992 45.850908) (end 122.504992 54.939408) (width 0.5) (layer B.Cu) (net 11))
 (segment (start 122.504992 54.939408) (end 119.9388 57.5056) (width 0.5) (layer B.Cu) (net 11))
 (segment (start 119.9388 57.5056) (end 117.2224 57.5056) (width 0.5) (layer B.Cu) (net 11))
 (segment (start 117.2224 57.5056) (end 116.8166 57.0998) (width 0.5) (layer B.Cu) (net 11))
 (segment (start 116.8166 57.0998) (end 116.8166 55.9498) (width 0.5) (layer B.Cu) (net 11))
 (segment (start 125.7046 38.7858) (end 125.7046 41.3258) (width 0.5) (layer B.Cu) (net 11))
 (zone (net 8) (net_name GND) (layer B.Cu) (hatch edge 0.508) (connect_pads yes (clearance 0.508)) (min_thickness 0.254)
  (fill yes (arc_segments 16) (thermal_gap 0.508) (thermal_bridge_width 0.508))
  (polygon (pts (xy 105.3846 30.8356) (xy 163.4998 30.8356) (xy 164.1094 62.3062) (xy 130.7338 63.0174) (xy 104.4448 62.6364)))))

